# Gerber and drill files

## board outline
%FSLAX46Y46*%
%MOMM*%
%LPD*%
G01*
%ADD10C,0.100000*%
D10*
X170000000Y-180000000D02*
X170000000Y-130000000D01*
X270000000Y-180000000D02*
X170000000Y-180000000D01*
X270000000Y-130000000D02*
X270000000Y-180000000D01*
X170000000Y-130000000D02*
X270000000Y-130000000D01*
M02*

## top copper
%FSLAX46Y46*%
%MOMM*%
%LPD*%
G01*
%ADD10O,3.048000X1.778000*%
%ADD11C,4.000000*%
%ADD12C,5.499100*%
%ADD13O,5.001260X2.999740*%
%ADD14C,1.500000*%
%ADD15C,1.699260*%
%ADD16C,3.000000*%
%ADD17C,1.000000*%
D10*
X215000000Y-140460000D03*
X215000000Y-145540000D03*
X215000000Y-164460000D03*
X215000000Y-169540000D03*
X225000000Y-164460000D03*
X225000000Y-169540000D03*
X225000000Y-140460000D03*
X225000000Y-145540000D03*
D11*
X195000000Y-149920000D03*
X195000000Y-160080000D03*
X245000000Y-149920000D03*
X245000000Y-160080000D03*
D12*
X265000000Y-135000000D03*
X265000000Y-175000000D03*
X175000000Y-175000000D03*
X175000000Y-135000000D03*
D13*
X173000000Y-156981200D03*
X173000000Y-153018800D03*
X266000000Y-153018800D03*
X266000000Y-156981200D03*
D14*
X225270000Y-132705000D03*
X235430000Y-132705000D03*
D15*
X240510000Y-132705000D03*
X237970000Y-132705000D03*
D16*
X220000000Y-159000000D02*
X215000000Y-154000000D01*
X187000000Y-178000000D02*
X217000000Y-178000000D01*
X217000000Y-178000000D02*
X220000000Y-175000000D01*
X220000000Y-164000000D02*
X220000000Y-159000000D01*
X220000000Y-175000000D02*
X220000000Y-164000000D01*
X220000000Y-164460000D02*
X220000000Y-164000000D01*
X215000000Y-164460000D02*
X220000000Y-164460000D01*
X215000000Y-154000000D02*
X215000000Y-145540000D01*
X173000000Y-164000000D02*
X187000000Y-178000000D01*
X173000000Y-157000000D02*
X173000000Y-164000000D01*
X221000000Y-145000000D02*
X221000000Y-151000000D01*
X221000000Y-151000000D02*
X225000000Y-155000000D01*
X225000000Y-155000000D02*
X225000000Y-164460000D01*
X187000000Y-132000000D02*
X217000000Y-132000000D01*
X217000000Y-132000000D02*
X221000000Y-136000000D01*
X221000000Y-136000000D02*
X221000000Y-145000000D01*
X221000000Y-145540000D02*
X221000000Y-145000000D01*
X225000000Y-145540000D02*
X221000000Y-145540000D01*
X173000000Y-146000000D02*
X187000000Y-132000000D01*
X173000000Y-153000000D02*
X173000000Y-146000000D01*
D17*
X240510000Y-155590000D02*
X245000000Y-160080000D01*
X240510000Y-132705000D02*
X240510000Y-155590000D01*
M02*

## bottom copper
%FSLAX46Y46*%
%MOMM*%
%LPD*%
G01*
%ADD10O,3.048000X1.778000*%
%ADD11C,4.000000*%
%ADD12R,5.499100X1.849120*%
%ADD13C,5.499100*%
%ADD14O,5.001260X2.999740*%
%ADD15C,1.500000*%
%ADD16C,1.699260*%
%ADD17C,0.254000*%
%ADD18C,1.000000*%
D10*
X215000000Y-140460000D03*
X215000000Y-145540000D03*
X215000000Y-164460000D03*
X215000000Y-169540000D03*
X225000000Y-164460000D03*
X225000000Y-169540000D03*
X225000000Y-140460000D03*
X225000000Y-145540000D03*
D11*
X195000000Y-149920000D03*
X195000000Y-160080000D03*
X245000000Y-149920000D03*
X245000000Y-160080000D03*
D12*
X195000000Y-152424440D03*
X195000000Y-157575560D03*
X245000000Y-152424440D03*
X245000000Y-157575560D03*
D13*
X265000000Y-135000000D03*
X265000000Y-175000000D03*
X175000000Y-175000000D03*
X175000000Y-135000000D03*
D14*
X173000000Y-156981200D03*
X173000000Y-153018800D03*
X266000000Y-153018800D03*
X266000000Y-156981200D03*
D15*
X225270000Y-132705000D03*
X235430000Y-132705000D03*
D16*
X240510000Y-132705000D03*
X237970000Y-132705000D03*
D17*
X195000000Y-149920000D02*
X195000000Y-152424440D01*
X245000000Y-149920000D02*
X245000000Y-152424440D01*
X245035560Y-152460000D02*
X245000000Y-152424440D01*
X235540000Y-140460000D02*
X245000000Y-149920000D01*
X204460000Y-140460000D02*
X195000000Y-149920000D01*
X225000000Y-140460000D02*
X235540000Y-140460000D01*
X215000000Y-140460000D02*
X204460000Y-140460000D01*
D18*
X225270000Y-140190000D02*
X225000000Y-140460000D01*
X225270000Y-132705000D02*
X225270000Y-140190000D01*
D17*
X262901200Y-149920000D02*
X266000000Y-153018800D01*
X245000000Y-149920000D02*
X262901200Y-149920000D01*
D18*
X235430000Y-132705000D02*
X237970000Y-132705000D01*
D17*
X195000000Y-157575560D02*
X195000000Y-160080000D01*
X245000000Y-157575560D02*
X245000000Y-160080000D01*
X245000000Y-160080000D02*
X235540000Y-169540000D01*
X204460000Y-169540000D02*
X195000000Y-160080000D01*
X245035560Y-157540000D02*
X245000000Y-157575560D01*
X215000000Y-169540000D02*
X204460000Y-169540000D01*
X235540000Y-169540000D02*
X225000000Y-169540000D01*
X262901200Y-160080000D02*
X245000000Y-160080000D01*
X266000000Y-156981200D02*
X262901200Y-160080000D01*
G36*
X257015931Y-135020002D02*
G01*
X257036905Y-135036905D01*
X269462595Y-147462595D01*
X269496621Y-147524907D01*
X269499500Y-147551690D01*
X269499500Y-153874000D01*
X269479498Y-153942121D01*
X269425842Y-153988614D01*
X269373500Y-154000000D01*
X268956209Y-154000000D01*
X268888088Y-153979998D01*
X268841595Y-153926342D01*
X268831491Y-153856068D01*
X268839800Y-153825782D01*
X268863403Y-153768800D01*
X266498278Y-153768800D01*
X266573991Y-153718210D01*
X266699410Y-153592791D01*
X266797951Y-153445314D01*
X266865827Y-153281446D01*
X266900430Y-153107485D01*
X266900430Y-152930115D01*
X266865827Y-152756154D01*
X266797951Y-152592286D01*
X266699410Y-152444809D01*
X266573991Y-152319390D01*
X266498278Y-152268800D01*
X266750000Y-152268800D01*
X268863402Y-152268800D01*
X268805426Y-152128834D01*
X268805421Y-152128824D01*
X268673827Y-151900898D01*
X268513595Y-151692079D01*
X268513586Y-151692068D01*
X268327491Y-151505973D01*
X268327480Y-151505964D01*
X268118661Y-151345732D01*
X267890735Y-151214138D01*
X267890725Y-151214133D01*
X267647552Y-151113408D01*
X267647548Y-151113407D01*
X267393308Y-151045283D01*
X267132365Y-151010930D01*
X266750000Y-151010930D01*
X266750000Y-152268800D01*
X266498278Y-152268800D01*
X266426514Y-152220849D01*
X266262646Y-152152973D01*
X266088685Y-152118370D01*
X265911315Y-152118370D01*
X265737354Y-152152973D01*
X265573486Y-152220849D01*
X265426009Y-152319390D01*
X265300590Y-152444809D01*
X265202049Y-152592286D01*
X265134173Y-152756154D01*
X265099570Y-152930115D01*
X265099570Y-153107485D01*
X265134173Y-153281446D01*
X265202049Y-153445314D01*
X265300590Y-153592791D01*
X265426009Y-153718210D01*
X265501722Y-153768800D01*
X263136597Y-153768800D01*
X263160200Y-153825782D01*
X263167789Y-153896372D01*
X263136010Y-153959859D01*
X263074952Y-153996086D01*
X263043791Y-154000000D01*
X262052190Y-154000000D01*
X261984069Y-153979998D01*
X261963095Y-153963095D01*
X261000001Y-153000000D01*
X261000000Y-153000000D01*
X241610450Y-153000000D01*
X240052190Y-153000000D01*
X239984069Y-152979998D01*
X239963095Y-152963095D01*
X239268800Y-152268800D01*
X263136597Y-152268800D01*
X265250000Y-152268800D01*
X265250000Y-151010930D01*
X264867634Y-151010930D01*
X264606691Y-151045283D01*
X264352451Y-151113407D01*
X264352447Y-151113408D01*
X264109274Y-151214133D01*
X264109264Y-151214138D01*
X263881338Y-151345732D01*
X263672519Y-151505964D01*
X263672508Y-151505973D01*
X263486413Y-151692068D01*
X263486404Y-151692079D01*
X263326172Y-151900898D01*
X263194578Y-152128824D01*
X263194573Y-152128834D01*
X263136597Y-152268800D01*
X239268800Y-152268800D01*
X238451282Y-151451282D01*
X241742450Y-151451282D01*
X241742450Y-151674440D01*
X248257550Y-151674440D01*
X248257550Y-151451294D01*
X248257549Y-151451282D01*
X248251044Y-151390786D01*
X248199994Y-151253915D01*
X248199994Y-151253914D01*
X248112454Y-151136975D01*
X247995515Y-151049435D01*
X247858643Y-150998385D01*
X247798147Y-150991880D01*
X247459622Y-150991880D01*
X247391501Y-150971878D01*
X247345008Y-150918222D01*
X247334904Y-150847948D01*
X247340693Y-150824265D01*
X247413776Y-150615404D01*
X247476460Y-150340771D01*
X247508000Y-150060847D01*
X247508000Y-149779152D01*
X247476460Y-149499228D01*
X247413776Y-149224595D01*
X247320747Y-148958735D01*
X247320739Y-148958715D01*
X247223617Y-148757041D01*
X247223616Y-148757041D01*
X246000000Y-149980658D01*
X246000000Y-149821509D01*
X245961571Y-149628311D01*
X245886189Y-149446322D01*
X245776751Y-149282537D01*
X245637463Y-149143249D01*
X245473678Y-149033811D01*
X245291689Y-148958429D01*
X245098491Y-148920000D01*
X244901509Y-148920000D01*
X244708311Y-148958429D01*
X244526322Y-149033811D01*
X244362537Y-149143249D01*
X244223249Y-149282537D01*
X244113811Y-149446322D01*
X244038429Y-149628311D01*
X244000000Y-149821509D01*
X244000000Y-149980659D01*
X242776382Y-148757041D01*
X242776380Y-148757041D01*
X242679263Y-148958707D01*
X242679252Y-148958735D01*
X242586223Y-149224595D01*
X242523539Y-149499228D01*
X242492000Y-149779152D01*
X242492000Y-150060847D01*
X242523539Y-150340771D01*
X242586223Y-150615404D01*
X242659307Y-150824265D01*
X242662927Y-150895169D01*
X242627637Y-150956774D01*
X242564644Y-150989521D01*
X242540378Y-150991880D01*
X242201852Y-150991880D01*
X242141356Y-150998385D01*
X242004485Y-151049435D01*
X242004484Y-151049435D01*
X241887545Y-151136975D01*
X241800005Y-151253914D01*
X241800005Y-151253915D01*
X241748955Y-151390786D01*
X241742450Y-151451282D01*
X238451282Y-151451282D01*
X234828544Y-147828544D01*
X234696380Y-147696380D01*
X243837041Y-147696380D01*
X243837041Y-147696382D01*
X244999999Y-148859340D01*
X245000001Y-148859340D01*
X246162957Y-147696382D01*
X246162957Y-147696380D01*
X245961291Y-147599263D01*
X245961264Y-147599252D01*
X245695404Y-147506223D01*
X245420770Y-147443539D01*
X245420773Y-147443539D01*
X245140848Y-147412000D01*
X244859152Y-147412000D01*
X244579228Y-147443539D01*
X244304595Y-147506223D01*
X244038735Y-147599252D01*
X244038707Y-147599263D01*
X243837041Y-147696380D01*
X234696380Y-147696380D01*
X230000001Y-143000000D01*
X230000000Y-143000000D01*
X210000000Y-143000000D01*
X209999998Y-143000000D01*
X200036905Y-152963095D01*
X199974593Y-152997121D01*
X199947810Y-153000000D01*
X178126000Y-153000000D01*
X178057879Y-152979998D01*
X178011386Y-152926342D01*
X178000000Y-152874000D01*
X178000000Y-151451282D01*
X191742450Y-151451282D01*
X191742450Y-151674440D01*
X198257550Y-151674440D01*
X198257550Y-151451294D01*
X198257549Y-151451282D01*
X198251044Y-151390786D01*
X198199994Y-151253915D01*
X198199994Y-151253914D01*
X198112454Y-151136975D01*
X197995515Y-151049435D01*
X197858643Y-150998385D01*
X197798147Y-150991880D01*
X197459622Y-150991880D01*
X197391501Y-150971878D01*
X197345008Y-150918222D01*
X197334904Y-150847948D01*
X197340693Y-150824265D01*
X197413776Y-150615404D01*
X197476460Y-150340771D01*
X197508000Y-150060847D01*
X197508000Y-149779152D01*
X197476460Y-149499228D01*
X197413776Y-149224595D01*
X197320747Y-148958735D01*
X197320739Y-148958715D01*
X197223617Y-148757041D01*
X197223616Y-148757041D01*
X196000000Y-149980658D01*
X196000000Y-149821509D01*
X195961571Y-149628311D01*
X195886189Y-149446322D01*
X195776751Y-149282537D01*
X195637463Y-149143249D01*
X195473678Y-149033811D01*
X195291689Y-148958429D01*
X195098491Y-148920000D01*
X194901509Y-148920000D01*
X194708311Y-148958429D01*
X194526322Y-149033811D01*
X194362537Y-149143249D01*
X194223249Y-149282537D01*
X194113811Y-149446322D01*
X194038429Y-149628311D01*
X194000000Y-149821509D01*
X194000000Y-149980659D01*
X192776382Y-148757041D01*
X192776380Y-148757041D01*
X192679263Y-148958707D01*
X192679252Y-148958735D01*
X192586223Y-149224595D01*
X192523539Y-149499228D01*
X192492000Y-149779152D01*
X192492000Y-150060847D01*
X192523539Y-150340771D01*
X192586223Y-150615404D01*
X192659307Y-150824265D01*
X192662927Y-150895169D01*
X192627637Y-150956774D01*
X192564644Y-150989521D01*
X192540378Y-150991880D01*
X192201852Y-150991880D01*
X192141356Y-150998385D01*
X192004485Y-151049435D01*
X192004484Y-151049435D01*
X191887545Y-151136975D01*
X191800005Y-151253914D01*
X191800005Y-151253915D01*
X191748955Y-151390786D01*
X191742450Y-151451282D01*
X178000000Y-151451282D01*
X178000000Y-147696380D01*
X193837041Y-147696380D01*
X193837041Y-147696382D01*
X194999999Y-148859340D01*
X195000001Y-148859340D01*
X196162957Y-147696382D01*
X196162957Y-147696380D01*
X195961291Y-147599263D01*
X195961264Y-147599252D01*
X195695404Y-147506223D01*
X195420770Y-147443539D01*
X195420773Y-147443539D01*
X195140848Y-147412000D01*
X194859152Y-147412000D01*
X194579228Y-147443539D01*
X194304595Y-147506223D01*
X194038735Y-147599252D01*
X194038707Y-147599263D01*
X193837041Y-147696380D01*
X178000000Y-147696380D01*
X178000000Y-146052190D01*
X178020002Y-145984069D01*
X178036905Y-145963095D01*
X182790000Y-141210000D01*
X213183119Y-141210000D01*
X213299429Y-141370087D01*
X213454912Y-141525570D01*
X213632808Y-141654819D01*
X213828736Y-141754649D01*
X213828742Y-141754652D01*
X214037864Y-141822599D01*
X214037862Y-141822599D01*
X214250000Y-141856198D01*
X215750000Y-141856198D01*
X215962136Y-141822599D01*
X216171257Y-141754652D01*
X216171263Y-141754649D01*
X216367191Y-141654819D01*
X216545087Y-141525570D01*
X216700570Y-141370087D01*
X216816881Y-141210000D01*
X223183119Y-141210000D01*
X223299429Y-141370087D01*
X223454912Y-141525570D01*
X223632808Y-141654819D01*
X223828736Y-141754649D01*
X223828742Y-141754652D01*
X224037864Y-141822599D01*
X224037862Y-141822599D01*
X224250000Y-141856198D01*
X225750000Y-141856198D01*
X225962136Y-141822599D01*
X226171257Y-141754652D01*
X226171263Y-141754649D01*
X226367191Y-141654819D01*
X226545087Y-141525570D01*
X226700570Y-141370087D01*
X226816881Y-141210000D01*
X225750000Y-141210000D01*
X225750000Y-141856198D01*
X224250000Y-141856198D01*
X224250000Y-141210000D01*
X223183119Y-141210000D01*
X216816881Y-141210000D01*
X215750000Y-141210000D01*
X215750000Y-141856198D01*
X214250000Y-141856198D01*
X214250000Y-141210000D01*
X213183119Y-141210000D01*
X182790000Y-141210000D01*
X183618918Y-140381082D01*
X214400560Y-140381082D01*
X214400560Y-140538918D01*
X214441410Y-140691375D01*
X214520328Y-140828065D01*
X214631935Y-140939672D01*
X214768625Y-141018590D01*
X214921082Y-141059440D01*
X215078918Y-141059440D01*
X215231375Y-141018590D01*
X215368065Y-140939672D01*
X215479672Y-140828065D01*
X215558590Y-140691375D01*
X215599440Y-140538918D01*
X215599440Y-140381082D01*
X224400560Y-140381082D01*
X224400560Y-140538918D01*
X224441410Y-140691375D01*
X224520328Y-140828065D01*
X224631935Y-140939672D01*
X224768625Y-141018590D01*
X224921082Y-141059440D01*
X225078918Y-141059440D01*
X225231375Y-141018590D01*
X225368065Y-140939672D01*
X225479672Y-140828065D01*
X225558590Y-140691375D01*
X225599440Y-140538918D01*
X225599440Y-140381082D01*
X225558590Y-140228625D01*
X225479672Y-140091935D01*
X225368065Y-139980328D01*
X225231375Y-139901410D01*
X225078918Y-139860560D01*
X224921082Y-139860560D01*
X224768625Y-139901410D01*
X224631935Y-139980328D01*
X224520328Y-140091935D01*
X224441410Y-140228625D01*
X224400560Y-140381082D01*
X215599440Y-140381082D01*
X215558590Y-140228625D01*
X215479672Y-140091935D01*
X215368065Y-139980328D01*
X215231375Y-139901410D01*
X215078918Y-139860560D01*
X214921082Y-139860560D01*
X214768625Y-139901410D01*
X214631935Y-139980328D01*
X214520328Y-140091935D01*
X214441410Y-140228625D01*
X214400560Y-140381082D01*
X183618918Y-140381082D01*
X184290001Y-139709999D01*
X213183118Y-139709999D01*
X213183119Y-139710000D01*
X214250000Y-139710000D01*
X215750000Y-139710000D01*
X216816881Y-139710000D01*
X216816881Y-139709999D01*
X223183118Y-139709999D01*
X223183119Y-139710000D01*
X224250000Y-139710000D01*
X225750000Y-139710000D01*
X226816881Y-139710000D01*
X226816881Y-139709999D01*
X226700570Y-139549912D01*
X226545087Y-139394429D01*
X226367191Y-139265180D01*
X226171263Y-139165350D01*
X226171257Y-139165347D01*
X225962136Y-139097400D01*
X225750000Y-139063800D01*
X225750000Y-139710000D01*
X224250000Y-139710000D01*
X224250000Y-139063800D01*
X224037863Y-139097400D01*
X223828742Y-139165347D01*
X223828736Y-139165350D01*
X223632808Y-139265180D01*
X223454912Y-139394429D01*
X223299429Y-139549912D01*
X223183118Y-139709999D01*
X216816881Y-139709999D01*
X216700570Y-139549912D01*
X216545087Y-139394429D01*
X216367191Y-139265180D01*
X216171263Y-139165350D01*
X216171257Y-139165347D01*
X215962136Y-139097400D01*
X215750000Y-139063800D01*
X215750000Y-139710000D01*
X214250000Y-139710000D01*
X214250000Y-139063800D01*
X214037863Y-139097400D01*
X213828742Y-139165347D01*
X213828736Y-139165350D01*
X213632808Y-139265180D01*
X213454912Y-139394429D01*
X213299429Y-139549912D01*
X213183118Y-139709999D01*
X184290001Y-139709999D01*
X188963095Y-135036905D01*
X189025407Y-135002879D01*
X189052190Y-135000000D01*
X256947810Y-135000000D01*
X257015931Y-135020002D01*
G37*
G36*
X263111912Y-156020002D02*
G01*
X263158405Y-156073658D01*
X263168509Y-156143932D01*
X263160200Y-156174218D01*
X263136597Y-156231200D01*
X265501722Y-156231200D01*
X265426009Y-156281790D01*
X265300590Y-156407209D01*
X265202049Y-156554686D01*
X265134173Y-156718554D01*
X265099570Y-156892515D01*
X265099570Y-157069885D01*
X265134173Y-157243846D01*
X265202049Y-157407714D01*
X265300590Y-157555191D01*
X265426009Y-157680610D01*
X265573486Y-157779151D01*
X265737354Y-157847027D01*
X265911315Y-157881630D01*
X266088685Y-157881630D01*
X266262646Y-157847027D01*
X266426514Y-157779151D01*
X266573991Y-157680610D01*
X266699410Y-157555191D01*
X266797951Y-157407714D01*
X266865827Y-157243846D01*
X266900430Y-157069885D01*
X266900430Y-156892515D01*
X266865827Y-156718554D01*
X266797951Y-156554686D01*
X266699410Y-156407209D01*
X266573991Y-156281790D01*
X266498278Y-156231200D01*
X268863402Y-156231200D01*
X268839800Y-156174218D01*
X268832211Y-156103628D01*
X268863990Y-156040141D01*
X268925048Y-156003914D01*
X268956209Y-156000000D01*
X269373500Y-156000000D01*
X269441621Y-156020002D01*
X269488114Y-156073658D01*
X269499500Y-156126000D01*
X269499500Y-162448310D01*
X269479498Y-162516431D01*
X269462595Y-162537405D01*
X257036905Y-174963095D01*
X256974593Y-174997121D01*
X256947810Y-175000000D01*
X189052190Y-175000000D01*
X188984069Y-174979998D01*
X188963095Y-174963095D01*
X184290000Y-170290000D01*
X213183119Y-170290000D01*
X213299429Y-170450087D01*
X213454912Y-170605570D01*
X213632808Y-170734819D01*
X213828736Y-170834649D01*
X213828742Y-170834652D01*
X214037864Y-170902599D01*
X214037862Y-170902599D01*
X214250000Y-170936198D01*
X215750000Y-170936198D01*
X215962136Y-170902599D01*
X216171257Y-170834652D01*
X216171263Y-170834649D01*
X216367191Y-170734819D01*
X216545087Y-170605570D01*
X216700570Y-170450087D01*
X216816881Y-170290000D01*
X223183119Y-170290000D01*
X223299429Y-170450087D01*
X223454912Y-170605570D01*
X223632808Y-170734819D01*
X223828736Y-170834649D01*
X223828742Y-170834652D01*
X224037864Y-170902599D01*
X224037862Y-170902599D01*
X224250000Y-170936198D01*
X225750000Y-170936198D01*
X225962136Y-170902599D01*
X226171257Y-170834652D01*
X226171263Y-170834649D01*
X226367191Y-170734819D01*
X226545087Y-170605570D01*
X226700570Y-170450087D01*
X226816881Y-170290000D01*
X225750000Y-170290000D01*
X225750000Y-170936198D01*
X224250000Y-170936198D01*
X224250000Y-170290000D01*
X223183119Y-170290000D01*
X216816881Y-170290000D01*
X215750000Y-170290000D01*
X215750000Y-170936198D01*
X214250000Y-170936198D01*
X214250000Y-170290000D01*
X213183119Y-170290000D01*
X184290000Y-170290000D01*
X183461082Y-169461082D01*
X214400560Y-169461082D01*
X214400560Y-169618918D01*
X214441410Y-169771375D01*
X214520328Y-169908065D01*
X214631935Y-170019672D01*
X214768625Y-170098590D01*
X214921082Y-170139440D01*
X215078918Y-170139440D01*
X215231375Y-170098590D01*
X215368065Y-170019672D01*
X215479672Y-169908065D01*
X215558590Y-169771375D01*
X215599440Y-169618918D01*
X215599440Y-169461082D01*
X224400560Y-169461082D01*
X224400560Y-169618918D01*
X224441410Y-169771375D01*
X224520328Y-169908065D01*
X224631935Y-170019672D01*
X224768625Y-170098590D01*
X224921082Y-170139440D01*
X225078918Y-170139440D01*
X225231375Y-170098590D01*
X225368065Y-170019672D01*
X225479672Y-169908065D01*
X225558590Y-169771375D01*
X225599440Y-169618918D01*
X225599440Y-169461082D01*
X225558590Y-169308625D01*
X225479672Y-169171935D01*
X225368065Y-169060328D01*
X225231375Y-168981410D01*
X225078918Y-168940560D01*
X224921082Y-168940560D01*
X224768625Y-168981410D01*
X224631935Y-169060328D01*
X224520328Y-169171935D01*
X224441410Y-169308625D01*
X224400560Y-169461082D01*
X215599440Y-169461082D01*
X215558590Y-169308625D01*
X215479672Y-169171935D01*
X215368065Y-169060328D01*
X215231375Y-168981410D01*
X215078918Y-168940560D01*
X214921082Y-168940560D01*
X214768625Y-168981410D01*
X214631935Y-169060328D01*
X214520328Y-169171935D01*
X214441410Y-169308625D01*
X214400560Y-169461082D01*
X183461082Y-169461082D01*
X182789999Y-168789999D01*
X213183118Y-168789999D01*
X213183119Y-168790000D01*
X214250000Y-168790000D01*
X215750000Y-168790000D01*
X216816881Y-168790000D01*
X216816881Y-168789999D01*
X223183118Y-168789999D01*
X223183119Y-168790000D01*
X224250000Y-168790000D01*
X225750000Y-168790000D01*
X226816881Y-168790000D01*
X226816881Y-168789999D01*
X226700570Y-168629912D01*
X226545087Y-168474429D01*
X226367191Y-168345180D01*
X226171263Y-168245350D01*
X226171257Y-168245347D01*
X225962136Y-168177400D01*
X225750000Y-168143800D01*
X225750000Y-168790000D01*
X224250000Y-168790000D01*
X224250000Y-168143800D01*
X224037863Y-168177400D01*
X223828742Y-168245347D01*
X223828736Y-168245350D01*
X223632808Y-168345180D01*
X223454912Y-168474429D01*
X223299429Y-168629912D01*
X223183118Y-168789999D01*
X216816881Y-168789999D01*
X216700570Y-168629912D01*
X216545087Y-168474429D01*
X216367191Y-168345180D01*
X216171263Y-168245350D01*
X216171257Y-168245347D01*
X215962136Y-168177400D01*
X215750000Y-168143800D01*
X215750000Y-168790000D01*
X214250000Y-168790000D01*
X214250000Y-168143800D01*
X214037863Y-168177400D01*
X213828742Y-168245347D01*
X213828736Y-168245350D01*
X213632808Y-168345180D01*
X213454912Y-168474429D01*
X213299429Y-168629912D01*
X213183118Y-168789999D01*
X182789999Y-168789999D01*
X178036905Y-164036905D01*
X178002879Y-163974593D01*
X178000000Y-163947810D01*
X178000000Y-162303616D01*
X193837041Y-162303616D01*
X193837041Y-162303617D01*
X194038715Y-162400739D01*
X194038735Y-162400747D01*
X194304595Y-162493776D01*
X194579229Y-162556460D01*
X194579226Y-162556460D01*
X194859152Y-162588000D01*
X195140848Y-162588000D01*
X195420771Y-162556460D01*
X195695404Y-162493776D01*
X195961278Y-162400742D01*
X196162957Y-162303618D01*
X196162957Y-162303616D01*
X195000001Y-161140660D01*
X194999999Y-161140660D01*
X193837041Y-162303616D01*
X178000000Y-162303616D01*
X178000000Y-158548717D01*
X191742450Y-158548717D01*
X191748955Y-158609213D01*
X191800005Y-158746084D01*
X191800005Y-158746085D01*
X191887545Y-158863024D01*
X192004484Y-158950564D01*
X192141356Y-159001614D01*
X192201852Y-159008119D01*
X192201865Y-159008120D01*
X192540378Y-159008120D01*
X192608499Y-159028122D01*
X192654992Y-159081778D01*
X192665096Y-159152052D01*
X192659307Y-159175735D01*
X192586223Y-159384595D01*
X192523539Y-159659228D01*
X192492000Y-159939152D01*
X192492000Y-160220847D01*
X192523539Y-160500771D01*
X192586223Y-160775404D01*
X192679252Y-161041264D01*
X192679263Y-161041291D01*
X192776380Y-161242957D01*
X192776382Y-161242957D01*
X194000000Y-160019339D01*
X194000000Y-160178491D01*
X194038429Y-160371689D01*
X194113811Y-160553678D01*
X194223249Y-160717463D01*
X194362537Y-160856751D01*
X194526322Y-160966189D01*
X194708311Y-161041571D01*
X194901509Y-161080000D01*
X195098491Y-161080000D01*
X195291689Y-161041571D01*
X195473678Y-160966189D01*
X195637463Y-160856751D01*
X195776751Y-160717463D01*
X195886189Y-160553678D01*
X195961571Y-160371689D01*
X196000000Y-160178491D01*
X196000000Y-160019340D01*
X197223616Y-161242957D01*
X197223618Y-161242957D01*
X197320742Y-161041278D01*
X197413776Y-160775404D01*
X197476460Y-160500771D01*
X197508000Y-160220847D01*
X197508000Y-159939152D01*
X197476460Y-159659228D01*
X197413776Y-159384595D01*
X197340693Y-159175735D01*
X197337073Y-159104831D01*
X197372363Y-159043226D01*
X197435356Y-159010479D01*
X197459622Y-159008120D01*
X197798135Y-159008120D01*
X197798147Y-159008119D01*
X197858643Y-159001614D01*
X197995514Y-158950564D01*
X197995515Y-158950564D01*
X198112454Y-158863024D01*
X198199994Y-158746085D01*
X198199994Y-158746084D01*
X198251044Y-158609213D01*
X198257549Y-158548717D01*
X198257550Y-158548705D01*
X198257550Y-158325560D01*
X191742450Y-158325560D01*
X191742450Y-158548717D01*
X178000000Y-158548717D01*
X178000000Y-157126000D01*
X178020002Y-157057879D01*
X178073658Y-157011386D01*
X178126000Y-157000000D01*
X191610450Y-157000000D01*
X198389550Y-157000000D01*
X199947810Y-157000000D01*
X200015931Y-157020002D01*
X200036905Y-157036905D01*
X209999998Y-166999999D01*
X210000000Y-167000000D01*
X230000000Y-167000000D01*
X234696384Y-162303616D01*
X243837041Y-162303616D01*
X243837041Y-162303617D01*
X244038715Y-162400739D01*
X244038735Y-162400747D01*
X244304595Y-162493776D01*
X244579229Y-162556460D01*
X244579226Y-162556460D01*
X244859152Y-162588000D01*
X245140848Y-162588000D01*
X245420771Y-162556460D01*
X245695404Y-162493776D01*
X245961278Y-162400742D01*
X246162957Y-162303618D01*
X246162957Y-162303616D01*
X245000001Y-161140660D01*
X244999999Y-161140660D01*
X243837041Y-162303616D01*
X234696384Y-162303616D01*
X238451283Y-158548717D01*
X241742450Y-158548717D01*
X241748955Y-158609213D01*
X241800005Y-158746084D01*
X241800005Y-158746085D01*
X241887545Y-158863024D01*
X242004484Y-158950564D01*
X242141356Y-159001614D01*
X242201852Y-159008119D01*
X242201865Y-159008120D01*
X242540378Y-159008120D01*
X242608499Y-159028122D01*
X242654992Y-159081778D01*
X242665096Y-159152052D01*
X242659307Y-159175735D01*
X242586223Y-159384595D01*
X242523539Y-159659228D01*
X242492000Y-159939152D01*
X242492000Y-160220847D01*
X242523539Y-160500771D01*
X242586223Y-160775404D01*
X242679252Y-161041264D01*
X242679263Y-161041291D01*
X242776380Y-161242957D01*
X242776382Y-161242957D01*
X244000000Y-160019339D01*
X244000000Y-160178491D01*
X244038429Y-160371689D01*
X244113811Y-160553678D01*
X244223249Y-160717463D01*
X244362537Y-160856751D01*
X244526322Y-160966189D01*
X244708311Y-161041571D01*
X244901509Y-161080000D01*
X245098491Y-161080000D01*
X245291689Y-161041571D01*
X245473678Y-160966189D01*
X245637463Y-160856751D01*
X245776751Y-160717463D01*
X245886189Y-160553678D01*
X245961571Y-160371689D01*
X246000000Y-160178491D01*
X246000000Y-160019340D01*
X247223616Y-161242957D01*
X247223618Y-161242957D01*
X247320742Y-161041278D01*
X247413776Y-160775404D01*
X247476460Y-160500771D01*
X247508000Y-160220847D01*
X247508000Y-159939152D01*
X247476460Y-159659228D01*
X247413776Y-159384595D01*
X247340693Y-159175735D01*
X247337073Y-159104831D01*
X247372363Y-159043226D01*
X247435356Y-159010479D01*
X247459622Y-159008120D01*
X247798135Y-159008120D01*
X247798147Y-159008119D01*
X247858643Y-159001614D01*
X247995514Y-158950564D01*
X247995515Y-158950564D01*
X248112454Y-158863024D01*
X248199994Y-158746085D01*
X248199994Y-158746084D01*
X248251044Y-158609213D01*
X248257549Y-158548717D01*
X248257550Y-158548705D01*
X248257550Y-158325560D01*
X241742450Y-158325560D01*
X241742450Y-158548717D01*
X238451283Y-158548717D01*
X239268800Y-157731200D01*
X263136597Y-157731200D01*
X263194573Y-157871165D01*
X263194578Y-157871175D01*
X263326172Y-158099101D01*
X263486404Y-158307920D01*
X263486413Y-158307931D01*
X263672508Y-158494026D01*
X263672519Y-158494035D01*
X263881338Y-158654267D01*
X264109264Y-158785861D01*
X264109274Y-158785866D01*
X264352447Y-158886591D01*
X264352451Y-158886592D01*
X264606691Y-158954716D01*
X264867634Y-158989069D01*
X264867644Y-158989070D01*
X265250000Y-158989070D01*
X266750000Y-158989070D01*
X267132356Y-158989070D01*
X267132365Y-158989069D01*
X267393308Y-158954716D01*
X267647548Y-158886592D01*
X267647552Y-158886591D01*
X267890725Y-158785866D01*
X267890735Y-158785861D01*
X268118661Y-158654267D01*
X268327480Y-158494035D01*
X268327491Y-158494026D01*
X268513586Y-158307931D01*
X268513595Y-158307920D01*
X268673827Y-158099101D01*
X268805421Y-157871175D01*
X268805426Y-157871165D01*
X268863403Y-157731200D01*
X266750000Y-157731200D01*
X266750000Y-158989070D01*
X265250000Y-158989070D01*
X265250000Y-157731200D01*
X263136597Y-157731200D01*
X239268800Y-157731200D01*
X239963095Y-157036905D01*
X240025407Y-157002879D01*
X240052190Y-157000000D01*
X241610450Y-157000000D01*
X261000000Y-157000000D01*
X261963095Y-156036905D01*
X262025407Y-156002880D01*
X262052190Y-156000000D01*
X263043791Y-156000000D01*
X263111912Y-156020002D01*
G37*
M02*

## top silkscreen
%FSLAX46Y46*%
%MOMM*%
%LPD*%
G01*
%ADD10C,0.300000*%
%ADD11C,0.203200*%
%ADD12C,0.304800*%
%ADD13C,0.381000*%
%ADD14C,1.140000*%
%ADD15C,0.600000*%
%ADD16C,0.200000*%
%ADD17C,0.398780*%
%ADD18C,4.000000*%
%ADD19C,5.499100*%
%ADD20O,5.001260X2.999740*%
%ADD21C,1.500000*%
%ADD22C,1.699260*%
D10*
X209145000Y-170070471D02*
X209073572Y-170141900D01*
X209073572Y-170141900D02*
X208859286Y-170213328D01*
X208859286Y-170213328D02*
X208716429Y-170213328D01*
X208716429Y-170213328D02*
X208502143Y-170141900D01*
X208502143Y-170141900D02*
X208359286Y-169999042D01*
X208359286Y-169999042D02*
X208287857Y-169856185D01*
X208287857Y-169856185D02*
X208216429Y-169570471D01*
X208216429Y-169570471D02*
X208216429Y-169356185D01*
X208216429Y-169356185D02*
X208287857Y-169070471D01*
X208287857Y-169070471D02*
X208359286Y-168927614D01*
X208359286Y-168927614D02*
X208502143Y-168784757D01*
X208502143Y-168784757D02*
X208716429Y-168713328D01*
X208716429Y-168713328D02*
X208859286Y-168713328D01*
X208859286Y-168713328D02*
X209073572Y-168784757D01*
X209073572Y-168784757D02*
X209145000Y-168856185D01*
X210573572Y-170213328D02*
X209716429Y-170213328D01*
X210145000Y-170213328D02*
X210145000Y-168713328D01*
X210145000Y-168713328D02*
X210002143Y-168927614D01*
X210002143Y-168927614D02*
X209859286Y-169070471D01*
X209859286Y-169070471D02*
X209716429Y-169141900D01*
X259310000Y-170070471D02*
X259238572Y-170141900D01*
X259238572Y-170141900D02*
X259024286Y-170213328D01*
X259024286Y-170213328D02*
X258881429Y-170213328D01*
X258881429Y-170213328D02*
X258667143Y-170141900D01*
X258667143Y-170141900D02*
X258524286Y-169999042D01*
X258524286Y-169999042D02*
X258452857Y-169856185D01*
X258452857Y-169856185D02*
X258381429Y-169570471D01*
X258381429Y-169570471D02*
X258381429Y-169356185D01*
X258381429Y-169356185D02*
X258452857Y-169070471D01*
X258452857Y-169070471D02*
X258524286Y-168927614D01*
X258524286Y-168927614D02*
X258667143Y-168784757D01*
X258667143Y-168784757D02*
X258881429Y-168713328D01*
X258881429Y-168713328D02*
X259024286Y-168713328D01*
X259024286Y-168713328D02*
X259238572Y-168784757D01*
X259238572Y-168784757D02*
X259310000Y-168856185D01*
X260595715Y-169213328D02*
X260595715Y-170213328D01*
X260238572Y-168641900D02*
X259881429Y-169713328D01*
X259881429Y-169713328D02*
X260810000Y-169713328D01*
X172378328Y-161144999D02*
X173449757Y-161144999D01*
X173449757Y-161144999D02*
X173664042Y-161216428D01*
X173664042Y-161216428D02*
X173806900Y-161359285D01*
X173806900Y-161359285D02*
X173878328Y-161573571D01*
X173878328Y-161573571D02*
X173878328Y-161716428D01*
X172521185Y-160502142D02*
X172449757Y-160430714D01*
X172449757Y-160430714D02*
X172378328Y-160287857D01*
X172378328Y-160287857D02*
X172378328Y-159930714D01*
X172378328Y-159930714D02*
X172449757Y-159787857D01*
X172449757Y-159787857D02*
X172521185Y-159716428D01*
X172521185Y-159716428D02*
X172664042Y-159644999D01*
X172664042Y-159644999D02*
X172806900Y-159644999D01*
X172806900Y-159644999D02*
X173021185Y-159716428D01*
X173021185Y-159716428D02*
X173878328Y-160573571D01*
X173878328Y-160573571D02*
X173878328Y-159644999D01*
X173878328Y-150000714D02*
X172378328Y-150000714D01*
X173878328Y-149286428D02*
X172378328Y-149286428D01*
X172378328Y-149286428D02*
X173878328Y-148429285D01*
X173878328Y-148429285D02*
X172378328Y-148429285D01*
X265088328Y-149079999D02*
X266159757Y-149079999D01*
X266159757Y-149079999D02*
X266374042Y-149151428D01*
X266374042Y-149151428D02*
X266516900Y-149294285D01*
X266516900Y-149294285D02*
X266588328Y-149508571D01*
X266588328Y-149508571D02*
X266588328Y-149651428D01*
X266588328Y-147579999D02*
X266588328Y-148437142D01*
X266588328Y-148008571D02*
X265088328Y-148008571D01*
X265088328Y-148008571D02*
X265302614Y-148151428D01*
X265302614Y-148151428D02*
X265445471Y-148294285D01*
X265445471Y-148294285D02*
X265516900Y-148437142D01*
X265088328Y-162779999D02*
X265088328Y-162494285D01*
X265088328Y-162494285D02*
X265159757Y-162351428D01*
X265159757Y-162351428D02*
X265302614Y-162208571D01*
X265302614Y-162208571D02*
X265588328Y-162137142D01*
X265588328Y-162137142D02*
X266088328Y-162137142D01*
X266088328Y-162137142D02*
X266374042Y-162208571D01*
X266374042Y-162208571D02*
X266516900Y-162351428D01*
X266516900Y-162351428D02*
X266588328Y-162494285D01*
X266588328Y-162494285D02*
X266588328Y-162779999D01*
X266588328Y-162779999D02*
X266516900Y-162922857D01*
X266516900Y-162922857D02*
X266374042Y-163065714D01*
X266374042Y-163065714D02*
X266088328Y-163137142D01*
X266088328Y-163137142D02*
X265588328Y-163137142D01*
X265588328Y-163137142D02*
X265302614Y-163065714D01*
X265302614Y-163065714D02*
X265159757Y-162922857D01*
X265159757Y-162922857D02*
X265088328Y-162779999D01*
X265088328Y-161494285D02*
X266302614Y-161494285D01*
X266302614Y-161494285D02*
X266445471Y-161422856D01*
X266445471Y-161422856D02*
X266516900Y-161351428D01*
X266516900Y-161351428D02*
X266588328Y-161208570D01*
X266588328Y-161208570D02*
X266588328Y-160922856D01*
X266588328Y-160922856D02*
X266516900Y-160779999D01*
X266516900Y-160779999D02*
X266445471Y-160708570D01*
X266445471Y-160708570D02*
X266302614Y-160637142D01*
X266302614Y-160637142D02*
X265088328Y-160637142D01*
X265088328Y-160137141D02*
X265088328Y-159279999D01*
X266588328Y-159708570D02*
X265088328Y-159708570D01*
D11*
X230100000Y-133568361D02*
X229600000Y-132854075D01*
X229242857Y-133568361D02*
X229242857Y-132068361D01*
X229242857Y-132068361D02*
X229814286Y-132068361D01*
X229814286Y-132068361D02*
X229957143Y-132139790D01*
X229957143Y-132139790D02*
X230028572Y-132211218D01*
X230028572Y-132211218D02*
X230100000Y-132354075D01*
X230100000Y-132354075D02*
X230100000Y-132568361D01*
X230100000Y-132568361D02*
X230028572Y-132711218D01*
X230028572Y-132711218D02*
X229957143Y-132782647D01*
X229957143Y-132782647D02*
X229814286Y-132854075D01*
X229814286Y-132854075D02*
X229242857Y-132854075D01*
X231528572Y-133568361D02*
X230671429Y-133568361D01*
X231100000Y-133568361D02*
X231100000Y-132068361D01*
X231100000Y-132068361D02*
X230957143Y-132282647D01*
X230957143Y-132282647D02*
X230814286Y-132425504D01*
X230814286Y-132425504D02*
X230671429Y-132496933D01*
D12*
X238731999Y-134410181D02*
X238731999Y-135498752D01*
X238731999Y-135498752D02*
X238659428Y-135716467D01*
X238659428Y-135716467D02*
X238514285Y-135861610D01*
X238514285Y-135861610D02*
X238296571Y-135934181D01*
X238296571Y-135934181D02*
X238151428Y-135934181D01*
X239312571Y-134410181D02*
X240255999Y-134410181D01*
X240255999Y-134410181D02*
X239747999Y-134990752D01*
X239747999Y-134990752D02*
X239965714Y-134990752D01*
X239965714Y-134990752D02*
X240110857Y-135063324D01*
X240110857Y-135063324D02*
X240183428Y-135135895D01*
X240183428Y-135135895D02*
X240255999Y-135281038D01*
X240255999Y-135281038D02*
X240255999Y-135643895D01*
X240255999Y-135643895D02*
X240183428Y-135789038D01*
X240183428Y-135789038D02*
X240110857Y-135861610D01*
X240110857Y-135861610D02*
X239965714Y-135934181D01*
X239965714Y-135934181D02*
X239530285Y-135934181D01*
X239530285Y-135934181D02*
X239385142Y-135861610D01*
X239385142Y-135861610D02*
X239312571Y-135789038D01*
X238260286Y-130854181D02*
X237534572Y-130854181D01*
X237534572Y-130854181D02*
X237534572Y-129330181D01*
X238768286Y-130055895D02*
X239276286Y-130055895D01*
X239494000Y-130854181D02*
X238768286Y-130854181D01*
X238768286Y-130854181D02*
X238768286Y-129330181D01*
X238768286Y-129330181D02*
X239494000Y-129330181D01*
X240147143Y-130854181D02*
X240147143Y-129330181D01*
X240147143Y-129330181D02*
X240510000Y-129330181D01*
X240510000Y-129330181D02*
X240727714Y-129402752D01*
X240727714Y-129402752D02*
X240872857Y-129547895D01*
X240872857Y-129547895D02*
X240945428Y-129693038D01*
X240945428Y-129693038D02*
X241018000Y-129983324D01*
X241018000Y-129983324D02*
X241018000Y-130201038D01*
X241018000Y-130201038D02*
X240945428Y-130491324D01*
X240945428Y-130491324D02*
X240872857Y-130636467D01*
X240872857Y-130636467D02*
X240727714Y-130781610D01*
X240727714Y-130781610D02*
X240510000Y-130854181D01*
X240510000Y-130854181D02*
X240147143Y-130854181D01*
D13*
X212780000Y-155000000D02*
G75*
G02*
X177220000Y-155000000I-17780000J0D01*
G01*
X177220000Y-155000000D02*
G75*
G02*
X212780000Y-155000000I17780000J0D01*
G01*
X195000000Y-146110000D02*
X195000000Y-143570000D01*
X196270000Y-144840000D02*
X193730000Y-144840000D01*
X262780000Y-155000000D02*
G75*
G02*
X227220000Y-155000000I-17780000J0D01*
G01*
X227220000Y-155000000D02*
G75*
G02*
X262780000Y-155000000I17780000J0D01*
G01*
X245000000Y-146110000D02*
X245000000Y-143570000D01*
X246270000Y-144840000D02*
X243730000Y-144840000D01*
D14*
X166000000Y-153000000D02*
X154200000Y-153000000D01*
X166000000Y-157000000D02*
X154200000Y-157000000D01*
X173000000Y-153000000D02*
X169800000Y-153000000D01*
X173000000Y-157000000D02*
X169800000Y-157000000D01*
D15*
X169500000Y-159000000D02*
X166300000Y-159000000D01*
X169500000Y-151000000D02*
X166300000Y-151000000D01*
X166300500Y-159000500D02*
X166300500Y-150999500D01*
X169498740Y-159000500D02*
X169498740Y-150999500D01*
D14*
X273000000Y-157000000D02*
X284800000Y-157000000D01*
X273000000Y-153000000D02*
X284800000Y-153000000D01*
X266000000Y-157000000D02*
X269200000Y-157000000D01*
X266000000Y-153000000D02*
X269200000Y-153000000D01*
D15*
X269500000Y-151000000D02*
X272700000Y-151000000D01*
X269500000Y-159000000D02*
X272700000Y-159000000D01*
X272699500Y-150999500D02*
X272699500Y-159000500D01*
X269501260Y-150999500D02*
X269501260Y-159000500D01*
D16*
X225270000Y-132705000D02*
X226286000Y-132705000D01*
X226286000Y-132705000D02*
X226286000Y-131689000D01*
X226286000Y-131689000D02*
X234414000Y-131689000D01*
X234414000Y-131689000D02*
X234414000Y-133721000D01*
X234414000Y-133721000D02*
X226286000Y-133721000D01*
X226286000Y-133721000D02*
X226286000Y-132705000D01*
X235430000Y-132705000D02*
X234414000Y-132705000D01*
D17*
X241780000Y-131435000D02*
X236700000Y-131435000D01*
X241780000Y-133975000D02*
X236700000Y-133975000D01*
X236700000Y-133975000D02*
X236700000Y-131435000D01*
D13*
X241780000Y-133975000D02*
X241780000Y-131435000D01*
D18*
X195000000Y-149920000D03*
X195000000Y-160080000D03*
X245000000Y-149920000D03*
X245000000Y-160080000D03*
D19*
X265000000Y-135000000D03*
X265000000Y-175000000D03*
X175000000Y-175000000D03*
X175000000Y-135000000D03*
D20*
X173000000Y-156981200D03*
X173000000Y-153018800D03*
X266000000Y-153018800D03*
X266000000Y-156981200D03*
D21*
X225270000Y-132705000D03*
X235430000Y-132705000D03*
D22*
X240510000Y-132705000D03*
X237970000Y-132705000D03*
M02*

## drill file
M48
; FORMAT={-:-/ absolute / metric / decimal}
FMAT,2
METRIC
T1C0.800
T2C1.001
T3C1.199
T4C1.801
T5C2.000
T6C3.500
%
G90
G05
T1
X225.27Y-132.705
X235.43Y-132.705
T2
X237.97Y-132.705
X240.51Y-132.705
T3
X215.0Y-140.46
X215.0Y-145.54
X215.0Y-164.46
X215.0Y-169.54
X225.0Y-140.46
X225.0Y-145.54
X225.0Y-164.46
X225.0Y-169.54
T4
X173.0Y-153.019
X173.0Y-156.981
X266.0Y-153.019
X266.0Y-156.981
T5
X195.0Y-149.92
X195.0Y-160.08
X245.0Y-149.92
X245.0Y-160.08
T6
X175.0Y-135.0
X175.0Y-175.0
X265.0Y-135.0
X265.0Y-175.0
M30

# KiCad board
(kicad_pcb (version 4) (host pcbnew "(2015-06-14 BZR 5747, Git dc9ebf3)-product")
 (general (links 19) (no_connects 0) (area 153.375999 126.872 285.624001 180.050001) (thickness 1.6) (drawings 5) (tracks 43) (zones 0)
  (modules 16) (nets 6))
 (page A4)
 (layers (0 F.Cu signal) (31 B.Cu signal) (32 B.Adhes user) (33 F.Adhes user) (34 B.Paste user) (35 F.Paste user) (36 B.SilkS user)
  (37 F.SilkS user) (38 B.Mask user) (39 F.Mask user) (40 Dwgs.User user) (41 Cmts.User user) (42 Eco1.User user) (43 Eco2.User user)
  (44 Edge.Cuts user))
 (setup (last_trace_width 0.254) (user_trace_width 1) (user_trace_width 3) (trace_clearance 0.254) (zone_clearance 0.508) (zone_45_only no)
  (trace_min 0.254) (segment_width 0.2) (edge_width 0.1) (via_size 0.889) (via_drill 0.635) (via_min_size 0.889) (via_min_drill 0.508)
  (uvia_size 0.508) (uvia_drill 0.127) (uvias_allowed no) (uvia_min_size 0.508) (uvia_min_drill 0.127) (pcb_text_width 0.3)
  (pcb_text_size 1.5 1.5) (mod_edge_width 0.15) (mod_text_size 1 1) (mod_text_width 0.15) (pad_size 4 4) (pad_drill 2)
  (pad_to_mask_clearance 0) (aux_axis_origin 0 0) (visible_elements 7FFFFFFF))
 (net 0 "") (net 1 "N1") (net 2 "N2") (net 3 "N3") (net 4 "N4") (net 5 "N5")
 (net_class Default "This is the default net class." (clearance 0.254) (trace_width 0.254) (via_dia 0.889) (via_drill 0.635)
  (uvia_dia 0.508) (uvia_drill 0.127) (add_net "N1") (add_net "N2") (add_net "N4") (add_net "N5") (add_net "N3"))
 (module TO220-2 (layer B.Cu) (at 215 143 180)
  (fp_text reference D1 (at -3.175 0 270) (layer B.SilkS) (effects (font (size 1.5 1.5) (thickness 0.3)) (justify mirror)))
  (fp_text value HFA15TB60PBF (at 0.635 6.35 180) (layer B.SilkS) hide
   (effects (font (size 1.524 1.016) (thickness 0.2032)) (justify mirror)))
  (pad 1 thru_hole oval (at 0 2.54 180) (size 3.048 1.778) (drill 1.19888) (layers *.Cu *.Mask B.SilkS) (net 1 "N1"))
  (pad 3 thru_hole oval (at 0 -2.54 180) (size 3.048 1.778) (drill 1.19888) (layers *.Cu *.Mask B.SilkS) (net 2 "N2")))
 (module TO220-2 (layer B.Cu) (at 215 167 180)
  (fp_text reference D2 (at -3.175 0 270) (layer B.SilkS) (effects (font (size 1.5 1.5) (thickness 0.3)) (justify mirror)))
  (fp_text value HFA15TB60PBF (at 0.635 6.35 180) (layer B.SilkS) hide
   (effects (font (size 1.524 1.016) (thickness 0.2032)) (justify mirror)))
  (pad 1 thru_hole oval (at 0 2.54 180) (size 3.048 1.778) (drill 1.19888) (layers *.Cu *.Mask B.SilkS) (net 2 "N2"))
  (pad 3 thru_hole oval (at 0 -2.54 180) (size 3.048 1.778) (drill 1.19888) (layers *.Cu *.Mask B.SilkS) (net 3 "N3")))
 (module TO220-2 (layer B.Cu) (at 225 167 180)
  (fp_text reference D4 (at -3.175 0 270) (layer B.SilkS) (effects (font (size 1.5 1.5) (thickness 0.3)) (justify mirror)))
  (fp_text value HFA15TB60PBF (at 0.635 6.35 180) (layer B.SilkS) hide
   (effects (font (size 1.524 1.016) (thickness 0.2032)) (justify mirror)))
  (pad 1 thru_hole oval (at 0 2.54 180) (size 3.048 1.778) (drill 1.19888) (layers *.Cu *.Mask B.SilkS) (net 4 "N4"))
  (pad 3 thru_hole oval (at 0 -2.54 180) (size 3.048 1.778) (drill 1.19888) (layers *.Cu *.Mask B.SilkS) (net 3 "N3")))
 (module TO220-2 (layer B.Cu) (at 225 143 180)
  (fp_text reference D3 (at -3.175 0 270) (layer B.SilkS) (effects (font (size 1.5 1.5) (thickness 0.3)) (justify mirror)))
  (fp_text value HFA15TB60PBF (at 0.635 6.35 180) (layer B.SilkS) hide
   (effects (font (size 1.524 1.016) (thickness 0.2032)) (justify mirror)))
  (pad 1 thru_hole oval (at 0 2.54 180) (size 3.048 1.778) (drill 1.19888) (layers *.Cu *.Mask B.SilkS) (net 1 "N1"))
  (pad 3 thru_hole oval (at 0 -2.54 180) (size 3.048 1.778) (drill 1.19888) (layers *.Cu *.Mask B.SilkS) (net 4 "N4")))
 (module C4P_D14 (layer F.Cu) (at 195 155 270)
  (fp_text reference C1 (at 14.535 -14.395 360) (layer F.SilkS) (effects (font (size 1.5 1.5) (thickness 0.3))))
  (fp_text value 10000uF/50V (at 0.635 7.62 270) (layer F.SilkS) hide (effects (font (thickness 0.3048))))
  (fp_circle (center 0 0) (end 17.78 0) (layer F.SilkS) (width 0.381))
  (fp_line (start -8.89 0) (end -11.43 0) (layer F.SilkS) (width 0.381))
  (fp_line (start -10.16 -1.27) (end -10.16 1.27) (layer F.SilkS) (width 0.381))
  (pad 1 thru_hole circle (at -5.08 0 270) (size 4 4) (drill 2) (layers *.Cu *.Mask F.SilkS) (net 1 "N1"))
  (pad 2 thru_hole circle (at 5.08 0 270) (size 4 4) (drill 2) (layers *.Cu *.Mask F.SilkS) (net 3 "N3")))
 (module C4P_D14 (layer F.Cu) (at 245 155 270)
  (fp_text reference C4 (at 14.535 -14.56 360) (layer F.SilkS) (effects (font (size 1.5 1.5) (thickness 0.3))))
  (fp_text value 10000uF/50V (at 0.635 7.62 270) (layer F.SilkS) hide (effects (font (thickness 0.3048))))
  (fp_circle (center 0 0) (end 17.78 0) (layer F.SilkS) (width 0.381))
  (fp_line (start -8.89 0) (end -11.43 0) (layer F.SilkS) (width 0.381))
  (fp_line (start -10.16 -1.27) (end -10.16 1.27) (layer F.SilkS) (width 0.381))
  (pad 1 thru_hole circle (at -5.08 0 270) (size 4 4) (drill 2) (layers *.Cu *.Mask F.SilkS) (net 1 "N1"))
  (pad 2 thru_hole circle (at 5.08 0 270) (size 4 4) (drill 2) (layers *.Cu *.Mask F.SilkS) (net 3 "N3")))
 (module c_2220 (layer B.Cu) (at 195 155 90)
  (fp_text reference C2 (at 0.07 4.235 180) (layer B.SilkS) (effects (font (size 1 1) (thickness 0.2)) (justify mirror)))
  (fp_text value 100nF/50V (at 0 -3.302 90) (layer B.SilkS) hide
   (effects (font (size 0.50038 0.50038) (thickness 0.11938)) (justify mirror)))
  (pad 1 smd rect (at 2.57556 0 90) (size 1.84912 5.4991) (layers B.Cu B.Paste B.Mask) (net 1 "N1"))
  (pad 2 smd rect (at -2.57556 0 90) (size 1.84912 5.4991) (layers B.Cu B.Paste B.Mask) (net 3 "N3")))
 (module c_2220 (layer B.Cu) (at 245 155 90)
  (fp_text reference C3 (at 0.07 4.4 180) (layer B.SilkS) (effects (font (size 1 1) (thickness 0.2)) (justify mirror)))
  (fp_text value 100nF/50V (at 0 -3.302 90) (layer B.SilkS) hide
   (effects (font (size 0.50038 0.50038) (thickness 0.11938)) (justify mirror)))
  (pad 1 smd rect (at 2.57556 0 90) (size 1.84912 5.4991) (layers B.Cu B.Paste B.Mask) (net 1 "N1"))
  (pad 2 smd rect (at -2.57556 0 90) (size 1.84912 5.4991) (layers B.Cu B.Paste B.Mask) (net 3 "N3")))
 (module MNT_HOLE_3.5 (layer F.Cu) (at 265 135)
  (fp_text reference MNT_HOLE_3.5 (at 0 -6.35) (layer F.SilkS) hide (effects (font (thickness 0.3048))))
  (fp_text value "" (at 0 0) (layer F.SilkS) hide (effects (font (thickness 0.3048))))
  (pad "" thru_hole circle (at 0 0) (size 5.4991 5.4991) (drill 3.50012) (layers *.Cu *.Mask F.SilkS)))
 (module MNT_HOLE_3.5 (layer F.Cu) (at 265 175)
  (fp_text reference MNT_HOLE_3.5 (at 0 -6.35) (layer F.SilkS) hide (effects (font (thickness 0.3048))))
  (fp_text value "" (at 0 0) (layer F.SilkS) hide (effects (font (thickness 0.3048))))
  (pad "" thru_hole circle (at 0 0) (size 5.4991 5.4991) (drill 3.50012) (layers *.Cu *.Mask F.SilkS)))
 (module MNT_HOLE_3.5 (layer F.Cu) (at 175 175)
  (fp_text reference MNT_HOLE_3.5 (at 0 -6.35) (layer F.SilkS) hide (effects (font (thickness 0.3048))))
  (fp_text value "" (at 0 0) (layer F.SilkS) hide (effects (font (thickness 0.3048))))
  (pad "" thru_hole circle (at 0 0) (size 5.4991 5.4991) (drill 3.50012) (layers *.Cu *.Mask F.SilkS)))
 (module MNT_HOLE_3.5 (layer F.Cu) (at 175 135)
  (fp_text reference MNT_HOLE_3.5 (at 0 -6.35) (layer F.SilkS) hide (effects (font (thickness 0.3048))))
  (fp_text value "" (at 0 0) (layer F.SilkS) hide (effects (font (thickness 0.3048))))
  (pad "" thru_hole circle (at 0 0) (size 5.4991 5.4991) (drill 3.50012) (layers *.Cu *.Mask F.SilkS)))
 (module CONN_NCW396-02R (layer F.Cu) (at 173 155 90)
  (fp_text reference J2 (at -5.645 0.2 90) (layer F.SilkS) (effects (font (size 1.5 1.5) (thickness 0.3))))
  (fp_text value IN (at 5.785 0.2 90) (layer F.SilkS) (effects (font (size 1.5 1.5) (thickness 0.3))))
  (fp_line (start 2 -7) (end 2 -18.8) (layer F.SilkS) (width 1.14))
  (fp_line (start -2 -7) (end -2 -18.8) (layer F.SilkS) (width 1.14))
  (fp_line (start 2 0) (end 2 -3.2) (layer F.SilkS) (width 1.14))
  (fp_line (start -2 0) (end -2 -3.2) (layer F.SilkS) (width 1.14))
  (fp_line (start -4 -3.5) (end -4 -6.7) (layer F.SilkS) (width 0.6))
  (fp_line (start 4 -3.5) (end 4 -6.7) (layer F.SilkS) (width 0.6))
  (fp_line (start -4.0005 -6.6995) (end 4.0005 -6.6995) (layer F.SilkS) (width 0.6))
  (fp_line (start -4.0005 -3.50126) (end 4.0005 -3.50126) (layer F.SilkS) (width 0.6))
  (pad 1 thru_hole oval (at -1.9812 0 90) (size 2.99974 5.00126) (drill 1.80086) (layers *.Cu *.Mask F.SilkS) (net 2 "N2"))
  (pad 2 thru_hole oval (at 1.9812 0 90) (size 2.99974 5.00126) (drill 1.80086) (layers *.Cu *.Mask F.SilkS) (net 4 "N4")))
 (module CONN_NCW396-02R (layer F.Cu) (at 266 155 270)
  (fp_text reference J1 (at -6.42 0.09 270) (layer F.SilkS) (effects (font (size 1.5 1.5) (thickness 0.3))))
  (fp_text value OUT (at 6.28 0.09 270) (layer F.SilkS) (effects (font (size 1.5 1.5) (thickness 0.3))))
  (fp_line (start 2 -7) (end 2 -18.8) (layer F.SilkS) (width 1.14))
  (fp_line (start -2 -7) (end -2 -18.8) (layer F.SilkS) (width 1.14))
  (fp_line (start 2 0) (end 2 -3.2) (layer F.SilkS) (width 1.14))
  (fp_line (start -2 0) (end -2 -3.2) (layer F.SilkS) (width 1.14))
  (fp_line (start -4 -3.5) (end -4 -6.7) (layer F.SilkS) (width 0.6))
  (fp_line (start 4 -3.5) (end 4 -6.7) (layer F.SilkS) (width 0.6))
  (fp_line (start -4.0005 -6.6995) (end 4.0005 -6.6995) (layer F.SilkS) (width 0.6))
  (fp_line (start -4.0005 -3.50126) (end 4.0005 -3.50126) (layer F.SilkS) (width 0.6))
  (pad 1 thru_hole oval (at -1.9812 0 270) (size 2.99974 5.00126) (drill 1.80086) (layers *.Cu *.Mask F.SilkS) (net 1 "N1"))
  (pad 2 thru_hole oval (at 1.9812 0 270) (size 2.99974 5.00126) (drill 1.80086) (layers *.Cu *.Mask F.SilkS) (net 3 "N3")))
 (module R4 (layer F.Cu) (at 230.35 132.705) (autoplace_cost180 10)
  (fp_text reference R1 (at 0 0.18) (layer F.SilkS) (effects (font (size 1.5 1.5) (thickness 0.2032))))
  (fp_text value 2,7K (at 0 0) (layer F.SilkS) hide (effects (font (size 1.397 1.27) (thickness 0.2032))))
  (fp_line (start -5.08 0) (end -4.064 0) (layer F.SilkS) (width 0.2))
  (fp_line (start -4.064 0) (end -4.064 -1.016) (layer F.SilkS) (width 0.2))
  (fp_line (start -4.064 -1.016) (end 4.064 -1.016) (layer F.SilkS) (width 0.2))
  (fp_line (start 4.064 -1.016) (end 4.064 1.016) (layer F.SilkS) (width 0.2))
  (fp_line (start 4.064 1.016) (end -4.064 1.016) (layer F.SilkS) (width 0.2))
  (fp_line (start -4.064 1.016) (end -4.064 0) (layer F.SilkS) (width 0.2))
  (fp_line (start 5.08 0) (end 4.064 0) (layer F.SilkS) (width 0.2))
  (pad 1 thru_hole circle (at -5.08 0) (size 1.5 1.5) (drill 0.8001) (layers *.Cu *.Mask F.SilkS) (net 1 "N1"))
  (pad 2 thru_hole circle (at 5.08 0) (size 1.5 1.5) (drill 0.8001) (layers *.Cu *.Mask F.SilkS) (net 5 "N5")))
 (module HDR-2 (layer F.Cu) (at 239.24 132.705 180)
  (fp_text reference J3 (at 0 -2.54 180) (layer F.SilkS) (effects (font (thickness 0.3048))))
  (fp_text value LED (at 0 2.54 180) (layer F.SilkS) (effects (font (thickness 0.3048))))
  (fp_line (start -2.54 1.27) (end 2.54 1.27) (layer F.SilkS) (width 0.39878))
  (fp_line (start -2.54 -1.27) (end 2.54 -1.27) (layer F.SilkS) (width 0.39878))
  (fp_line (start 2.54 -1.27) (end 2.54 1.27) (layer F.SilkS) (width 0.39878))
  (fp_line (start -2.54 -1.27) (end -2.54 1.27) (layer F.SilkS) (width 0.381))
  (pad 1 thru_hole circle (at -1.27 0 180) (size 1.69926 1.69926) (drill 1.00076) (layers *.Cu *.Mask F.SilkS) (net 3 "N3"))
  (pad 2 thru_hole circle (at 1.27 0 180) (size 1.69926 1.69926) (drill 1.00076) (layers *.Cu *.Mask F.SilkS) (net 5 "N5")))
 (gr_line (start 170 180) (end 170 130) (angle 90) (layer Edge.Cuts) (width 0.1))
 (gr_line (start 270 180) (end 170 180) (angle 90) (layer Edge.Cuts) (width 0.1))
 (gr_line (start 270 130) (end 270 180) (angle 90) (layer Edge.Cuts) (width 0.1))
 (gr_line (start 170 130) (end 270 130) (angle 90) (layer Edge.Cuts) (width 0.1))
 (segment (start 195 149.92) (end 195 152.42444) (width 0.254) (layer B.Cu) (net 1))
 (segment (start 245 149.92) (end 245 152.42444) (width 0.254) (layer B.Cu) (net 1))
 (segment (start 245.03556 152.46) (end 245 152.42444) (width 0.254) (layer B.Cu) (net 1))
 (segment (start 235.54 140.46) (end 245 149.92) (width 0.254) (layer B.Cu) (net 1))
 (segment (start 204.46 140.46) (end 195 149.92) (width 0.254) (layer B.Cu) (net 1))
 (segment (start 225 140.46) (end 235.54 140.46) (width 0.254) (layer B.Cu) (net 1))
 (segment (start 215 140.46) (end 204.46 140.46) (width 0.254) (layer B.Cu) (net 1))
 (segment (start 225.27 140.19) (end 225 140.46) (width 1) (layer B.Cu) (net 1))
 (segment (start 225.27 132.705) (end 225.27 140.19) (width 1) (layer B.Cu) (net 1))
 (segment (start 262.9012 149.92) (end 266 153.0188) (width 0.254) (layer B.Cu) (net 1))
 (segment (start 245 149.92) (end 262.9012 149.92) (width 0.254) (layer B.Cu) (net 1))
 (segment (start 220 159) (end 215 154) (width 3) (layer F.Cu) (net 2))
 (segment (start 187 178) (end 217 178) (width 3) (layer F.Cu) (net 2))
 (segment (start 217 178) (end 220 175) (width 3) (layer F.Cu) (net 2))
 (segment (start 220 164) (end 220 159) (width 3) (layer F.Cu) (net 2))
 (segment (start 220 175) (end 220 164) (width 3) (layer F.Cu) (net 2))
 (segment (start 220 164.46) (end 220 164) (width 3) (layer F.Cu) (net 2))
 (segment (start 215 164.46) (end 220 164.46) (width 3) (layer F.Cu) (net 2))
 (segment (start 215 154) (end 215 145.54) (width 3) (layer F.Cu) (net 2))
 (segment (start 173 164) (end 187 178) (width 3) (layer F.Cu) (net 2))
 (segment (start 173 157) (end 173 164) (width 3) (layer F.Cu) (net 2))
 (segment (start 221 145) (end 221 151) (width 3) (layer F.Cu) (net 4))
 (segment (start 221 151) (end 225 155) (width 3) (layer F.Cu) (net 4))
 (segment (start 225 155) (end 225 164.46) (width 3) (layer F.Cu) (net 4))
 (segment (start 187 132) (end 217 132) (width 3) (layer F.Cu) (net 4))
 (segment (start 217 132) (end 221 136) (width 3) (layer F.Cu) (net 4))
 (segment (start 221 136) (end 221 145) (width 3) (layer F.Cu) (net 4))
 (segment (start 221 145.54) (end 221 145) (width 3) (layer F.Cu) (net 4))
 (segment (start 225 145.54) (end 221 145.54) (width 3) (layer F.Cu) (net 4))
 (segment (start 173 146) (end 187 132) (width 3) (layer F.Cu) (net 4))
 (segment (start 173 153) (end 173 146) (width 3) (layer F.Cu) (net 4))
 (segment (start 235.43 132.705) (end 237.97 132.705) (width 1) (layer B.Cu) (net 5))
 (segment (start 195 157.57556) (end 195 160.08) (width 0.254) (layer B.Cu) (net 3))
 (segment (start 245 157.57556) (end 245 160.08) (width 0.254) (layer B.Cu) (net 3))
 (segment (start 245 160.08) (end 235.54 169.54) (width 0.254) (layer B.Cu) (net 3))
 (segment (start 204.46 169.54) (end 195 160.08) (width 0.254) (layer B.Cu) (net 3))
 (segment (start 245.03556 157.54) (end 245 157.57556) (width 0.254) (layer B.Cu) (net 3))
 (segment (start 215 169.54) (end 204.46 169.54) (width 0.254) (layer B.Cu) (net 3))
 (segment (start 235.54 169.54) (end 225 169.54) (width 0.254) (layer B.Cu) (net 3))
 (segment (start 240.51 155.59) (end 245 160.08) (width 1) (layer F.Cu) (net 3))
 (segment (start 240.51 132.705) (end 240.51 155.59) (width 1) (layer F.Cu) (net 3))
 (segment (start 262.9012 160.08) (end 245 160.08) (width 0.254) (layer B.Cu) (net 3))
 (segment (start 266 156.9812) (end 262.9012 160.08) (width 0.254) (layer B.Cu) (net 3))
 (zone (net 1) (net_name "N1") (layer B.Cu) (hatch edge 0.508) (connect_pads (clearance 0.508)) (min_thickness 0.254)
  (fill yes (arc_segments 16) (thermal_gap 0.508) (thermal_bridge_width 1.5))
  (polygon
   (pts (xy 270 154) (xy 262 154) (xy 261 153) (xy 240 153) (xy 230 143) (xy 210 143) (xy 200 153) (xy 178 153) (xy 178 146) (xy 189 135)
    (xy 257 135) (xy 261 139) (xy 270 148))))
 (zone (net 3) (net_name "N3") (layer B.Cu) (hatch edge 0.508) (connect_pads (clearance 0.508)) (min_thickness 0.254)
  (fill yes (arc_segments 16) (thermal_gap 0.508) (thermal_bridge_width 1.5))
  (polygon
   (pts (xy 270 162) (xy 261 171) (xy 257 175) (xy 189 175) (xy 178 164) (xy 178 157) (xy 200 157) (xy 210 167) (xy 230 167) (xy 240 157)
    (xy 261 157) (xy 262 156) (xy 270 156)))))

